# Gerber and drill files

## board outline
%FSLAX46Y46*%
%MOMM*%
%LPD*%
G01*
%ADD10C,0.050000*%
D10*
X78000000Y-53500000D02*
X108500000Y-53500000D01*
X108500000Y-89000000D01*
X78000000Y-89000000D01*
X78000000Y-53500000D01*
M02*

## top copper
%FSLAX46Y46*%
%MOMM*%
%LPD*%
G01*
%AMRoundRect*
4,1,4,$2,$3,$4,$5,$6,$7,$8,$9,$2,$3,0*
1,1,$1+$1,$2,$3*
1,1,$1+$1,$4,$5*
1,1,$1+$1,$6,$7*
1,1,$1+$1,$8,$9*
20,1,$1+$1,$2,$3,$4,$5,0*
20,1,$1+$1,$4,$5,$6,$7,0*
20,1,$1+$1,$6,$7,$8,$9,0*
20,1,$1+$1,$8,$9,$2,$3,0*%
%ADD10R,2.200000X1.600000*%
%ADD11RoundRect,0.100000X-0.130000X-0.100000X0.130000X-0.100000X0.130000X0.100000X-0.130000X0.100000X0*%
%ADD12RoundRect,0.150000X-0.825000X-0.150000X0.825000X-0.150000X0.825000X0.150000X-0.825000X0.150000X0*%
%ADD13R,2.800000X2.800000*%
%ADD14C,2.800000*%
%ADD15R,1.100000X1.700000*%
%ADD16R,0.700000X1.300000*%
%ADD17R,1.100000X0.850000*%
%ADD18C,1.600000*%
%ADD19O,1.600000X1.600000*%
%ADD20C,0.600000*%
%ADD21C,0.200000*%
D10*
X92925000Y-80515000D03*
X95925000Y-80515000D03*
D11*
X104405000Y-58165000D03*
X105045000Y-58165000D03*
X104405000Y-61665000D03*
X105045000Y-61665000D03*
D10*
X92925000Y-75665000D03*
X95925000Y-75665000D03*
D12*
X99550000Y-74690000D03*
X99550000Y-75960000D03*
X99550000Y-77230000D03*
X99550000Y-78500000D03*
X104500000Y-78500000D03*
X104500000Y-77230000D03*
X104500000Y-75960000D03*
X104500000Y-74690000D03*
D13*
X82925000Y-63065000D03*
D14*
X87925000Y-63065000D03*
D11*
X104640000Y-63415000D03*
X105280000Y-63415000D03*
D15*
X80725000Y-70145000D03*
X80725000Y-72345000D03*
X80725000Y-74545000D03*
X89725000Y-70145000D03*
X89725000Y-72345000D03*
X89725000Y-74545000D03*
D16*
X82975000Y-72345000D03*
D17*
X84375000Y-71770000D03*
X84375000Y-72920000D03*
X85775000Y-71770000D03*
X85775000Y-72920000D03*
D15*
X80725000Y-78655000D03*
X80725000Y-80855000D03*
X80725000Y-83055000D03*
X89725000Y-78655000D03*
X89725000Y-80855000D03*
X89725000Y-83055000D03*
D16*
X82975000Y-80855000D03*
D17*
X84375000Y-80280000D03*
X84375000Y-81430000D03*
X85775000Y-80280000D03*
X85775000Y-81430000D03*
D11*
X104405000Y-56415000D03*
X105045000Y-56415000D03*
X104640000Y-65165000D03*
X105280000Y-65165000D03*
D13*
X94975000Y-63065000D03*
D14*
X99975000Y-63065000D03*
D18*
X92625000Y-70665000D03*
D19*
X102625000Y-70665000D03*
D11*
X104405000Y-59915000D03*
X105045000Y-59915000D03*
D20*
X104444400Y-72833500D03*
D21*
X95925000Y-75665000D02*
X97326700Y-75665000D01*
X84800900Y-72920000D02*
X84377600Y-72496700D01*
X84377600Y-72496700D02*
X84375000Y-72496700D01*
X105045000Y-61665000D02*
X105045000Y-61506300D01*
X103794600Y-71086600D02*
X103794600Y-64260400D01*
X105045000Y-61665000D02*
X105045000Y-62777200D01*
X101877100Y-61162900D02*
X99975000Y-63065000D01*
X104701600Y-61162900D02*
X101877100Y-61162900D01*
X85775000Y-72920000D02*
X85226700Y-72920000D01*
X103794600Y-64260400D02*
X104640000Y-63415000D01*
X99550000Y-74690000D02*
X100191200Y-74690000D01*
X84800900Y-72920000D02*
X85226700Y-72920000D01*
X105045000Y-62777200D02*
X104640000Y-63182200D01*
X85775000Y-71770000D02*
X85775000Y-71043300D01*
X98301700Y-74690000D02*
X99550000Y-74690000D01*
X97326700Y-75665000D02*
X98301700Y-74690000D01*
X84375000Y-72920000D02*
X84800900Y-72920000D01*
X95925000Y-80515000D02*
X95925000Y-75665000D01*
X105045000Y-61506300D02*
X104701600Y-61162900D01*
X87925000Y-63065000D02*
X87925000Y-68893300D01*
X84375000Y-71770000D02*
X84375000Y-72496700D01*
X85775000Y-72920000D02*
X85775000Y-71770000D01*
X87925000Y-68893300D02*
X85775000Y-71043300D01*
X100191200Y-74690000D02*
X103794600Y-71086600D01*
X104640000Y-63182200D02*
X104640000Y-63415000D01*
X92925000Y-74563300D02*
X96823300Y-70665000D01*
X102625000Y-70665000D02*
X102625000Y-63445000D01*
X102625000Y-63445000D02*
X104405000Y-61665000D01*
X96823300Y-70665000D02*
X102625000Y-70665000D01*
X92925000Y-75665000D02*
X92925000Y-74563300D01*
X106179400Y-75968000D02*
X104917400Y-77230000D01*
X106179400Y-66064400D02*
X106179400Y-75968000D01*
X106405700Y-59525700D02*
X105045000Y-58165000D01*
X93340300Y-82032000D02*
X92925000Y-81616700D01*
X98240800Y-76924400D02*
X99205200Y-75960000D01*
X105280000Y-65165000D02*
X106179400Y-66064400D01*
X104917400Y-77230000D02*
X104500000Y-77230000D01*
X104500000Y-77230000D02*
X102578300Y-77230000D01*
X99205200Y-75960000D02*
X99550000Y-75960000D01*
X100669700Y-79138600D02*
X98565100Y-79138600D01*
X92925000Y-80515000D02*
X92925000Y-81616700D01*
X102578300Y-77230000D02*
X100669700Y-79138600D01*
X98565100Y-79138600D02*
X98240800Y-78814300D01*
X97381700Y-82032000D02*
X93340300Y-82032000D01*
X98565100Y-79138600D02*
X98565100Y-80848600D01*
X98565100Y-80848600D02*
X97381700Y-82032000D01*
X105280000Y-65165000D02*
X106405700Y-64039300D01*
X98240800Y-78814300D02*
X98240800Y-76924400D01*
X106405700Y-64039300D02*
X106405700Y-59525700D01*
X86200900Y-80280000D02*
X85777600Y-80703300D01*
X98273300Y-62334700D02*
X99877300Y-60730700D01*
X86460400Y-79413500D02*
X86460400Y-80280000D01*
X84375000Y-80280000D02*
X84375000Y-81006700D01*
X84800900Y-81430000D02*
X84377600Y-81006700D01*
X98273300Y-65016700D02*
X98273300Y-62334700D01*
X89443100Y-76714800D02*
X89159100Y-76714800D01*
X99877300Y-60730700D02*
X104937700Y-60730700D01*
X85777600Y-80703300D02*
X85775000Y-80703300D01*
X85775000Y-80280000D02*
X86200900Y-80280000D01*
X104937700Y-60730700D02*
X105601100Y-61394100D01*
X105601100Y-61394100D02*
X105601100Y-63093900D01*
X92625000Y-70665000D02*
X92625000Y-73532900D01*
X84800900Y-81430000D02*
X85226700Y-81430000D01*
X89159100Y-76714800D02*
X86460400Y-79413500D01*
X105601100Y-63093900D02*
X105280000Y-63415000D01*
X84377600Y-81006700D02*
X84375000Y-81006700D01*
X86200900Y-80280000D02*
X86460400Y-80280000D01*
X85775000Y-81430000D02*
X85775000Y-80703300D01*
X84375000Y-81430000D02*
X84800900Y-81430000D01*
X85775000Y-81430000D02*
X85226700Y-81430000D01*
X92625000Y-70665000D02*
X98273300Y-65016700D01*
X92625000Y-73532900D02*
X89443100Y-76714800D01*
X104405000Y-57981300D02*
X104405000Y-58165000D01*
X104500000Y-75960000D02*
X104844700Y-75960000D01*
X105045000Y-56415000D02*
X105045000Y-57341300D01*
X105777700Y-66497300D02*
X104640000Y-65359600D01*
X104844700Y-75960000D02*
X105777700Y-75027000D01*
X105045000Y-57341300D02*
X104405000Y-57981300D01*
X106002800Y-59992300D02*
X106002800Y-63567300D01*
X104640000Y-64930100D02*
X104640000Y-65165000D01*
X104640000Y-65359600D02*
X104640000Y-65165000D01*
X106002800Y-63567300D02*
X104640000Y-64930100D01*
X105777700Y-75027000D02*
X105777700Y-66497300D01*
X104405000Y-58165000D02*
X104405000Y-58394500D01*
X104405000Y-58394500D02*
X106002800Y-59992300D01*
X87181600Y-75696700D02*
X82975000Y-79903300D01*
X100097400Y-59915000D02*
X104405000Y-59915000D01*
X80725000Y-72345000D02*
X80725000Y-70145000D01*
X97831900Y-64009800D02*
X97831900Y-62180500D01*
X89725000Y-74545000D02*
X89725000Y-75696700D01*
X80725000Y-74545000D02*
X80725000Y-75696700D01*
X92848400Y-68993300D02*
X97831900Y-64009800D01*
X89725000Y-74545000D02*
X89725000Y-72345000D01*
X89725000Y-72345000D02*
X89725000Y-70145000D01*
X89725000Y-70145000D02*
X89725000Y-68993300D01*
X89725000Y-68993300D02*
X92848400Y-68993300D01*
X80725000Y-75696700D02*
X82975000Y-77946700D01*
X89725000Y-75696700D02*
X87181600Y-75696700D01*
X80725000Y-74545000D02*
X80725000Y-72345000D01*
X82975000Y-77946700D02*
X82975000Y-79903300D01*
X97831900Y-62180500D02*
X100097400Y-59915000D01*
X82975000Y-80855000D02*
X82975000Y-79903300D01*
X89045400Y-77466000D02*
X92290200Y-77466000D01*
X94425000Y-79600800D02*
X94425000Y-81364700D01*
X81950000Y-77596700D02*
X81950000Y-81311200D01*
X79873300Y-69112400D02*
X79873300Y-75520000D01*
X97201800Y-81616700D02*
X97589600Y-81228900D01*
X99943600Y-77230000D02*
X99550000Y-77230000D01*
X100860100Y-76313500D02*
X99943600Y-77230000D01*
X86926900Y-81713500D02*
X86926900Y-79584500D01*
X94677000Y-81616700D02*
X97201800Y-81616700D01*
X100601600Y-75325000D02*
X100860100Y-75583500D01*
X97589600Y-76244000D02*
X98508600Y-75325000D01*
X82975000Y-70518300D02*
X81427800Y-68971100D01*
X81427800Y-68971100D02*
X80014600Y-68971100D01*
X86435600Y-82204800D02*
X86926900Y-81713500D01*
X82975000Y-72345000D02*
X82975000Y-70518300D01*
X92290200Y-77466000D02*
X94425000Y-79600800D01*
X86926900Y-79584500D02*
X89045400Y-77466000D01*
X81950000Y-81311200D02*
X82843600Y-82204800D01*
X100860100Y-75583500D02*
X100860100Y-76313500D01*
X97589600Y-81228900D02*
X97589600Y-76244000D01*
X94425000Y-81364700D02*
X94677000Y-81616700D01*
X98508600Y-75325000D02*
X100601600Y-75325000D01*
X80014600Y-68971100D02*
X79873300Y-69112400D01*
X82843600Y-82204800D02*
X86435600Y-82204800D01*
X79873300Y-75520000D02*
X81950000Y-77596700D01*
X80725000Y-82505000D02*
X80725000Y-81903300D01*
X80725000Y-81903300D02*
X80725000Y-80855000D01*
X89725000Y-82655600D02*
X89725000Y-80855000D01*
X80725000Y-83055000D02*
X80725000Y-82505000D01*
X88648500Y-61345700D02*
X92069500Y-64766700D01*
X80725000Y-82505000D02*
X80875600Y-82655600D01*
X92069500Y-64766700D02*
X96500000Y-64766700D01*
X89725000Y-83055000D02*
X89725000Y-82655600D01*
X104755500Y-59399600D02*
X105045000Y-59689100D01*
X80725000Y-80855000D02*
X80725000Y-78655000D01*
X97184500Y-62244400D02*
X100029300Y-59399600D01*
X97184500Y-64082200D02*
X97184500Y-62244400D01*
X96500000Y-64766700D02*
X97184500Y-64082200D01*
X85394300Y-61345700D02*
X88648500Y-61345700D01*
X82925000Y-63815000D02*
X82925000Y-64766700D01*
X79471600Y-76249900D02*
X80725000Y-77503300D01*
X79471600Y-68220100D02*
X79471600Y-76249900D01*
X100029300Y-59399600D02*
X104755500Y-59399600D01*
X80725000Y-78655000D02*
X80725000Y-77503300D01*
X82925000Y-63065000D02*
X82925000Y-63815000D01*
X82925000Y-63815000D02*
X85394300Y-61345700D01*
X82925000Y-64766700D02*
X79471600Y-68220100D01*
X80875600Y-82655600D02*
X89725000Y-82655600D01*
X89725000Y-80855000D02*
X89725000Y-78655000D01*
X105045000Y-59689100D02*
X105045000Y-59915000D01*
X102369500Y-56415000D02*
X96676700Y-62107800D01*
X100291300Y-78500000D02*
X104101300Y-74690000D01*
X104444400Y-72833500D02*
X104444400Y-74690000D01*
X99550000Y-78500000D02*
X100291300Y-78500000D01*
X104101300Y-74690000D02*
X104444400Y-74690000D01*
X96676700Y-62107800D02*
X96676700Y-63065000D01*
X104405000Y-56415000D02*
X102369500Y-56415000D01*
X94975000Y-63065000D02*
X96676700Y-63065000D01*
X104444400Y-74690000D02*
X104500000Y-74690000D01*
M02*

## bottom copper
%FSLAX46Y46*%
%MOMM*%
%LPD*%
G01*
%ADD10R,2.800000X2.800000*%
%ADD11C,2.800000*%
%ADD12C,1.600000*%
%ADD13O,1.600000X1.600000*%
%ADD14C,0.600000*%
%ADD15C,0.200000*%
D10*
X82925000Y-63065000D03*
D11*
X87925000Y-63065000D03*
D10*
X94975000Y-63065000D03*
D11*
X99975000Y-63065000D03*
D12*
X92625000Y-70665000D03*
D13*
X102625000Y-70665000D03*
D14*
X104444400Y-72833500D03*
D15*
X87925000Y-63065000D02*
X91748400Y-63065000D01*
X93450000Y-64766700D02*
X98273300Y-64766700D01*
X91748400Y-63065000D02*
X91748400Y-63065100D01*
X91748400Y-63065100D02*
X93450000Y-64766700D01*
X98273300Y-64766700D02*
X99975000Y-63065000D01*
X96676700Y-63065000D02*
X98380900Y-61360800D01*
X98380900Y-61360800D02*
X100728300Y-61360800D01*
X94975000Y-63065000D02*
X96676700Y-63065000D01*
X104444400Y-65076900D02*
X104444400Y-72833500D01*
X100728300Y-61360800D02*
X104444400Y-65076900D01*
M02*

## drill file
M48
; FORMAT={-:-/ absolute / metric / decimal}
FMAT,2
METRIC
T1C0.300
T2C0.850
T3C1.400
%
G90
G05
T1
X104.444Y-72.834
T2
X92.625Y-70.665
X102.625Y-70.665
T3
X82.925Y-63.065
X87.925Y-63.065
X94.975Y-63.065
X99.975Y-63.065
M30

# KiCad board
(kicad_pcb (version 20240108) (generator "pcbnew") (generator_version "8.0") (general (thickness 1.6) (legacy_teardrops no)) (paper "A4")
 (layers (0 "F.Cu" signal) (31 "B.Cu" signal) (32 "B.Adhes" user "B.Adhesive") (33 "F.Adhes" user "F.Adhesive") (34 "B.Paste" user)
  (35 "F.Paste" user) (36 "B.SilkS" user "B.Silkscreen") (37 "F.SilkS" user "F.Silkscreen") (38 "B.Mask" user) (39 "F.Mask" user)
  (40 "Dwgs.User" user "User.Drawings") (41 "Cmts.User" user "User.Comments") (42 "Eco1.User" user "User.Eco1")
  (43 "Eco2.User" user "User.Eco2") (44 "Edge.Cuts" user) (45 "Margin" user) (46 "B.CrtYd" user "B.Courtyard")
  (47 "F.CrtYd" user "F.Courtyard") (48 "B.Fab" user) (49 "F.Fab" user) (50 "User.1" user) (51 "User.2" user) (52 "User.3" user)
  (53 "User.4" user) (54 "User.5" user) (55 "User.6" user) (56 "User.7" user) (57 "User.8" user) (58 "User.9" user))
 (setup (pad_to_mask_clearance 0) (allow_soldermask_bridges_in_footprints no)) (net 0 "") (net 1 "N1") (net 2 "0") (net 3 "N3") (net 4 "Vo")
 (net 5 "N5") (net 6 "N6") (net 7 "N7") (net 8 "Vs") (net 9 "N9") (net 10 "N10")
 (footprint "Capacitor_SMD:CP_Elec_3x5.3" (layer "F.Cu") (at 94.425 80.515)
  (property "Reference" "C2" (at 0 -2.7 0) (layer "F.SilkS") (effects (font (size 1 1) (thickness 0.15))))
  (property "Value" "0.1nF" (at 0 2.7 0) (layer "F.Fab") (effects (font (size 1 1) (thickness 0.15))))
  (pad "1" smd rect (at -1.5 0) (size 2.2 1.6) (layers "F.Cu" "F.Paste" "F.Mask") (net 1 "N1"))
  (pad "2" smd rect (at 1.5 0) (size 2.2 1.6) (layers "F.Cu" "F.Paste" "F.Mask") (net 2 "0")))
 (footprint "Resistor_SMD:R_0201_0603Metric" (layer "F.Cu") (at 104.725 58.165)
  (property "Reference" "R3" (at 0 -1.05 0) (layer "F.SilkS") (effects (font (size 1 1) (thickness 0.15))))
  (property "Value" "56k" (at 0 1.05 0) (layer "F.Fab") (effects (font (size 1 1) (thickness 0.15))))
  (pad "" smd roundrect (at -0.345 0) (size 0.318 0.36) (layers "F.Paste") (roundrect_rratio 0.25))
  (pad "" smd roundrect (at 0.345 0) (size 0.318 0.36) (layers "F.Paste") (roundrect_rratio 0.25))
  (pad "1" smd roundrect (at -0.32 0) (size 0.46 0.4) (layers "F.Cu" "F.Mask") (roundrect_rratio 0.25) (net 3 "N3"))
  (pad "2" smd roundrect (at 0.32 0) (size 0.46 0.4) (layers "F.Cu" "F.Mask") (roundrect_rratio 0.25) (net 1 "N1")))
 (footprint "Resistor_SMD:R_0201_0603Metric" (layer "F.Cu") (at 104.725 61.665)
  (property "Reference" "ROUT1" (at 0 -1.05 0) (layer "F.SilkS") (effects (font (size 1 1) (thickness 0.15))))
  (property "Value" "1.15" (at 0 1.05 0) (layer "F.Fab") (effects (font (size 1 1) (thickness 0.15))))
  (pad "" smd roundrect (at -0.345 0) (size 0.318 0.36) (layers "F.Paste") (roundrect_rratio 0.25))
  (pad "" smd roundrect (at 0.345 0) (size 0.318 0.36) (layers "F.Paste") (roundrect_rratio 0.25))
  (pad "1" smd roundrect (at -0.32 0) (size 0.46 0.4) (layers "F.Cu" "F.Mask") (roundrect_rratio 0.25) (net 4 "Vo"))
  (pad "2" smd roundrect (at 0.32 0) (size 0.46 0.4) (layers "F.Cu" "F.Mask") (roundrect_rratio 0.25) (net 2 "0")))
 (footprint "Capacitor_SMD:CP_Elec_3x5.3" (layer "F.Cu") (at 94.425 75.665)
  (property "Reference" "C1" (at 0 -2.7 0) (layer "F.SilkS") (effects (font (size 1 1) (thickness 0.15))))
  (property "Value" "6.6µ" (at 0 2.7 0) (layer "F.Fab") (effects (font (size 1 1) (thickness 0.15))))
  (pad "1" smd rect (at -1.5 0) (size 2.2 1.6) (layers "F.Cu" "F.Paste" "F.Mask") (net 4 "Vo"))
  (pad "2" smd rect (at 1.5 0) (size 2.2 1.6) (layers "F.Cu" "F.Paste" "F.Mask") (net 2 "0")))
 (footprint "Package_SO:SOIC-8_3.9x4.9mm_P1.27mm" (layer "F.Cu") (at 102.025 76.595)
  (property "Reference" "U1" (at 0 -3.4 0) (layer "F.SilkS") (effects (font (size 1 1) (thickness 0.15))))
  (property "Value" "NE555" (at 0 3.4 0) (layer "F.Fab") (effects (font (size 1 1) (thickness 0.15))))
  (pad "1" smd roundrect (at -2.475 -1.905) (size 1.95 0.6) (layers "F.Cu" "F.Paste" "F.Mask") (roundrect_rratio 0.25) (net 2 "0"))
  (pad "2" smd roundrect (at -2.475 -0.635) (size 1.95 0.6) (layers "F.Cu" "F.Paste" "F.Mask") (roundrect_rratio 0.25) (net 1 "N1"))
  (pad "3" smd roundrect (at -2.475 0.635) (size 1.95 0.6) (layers "F.Cu" "F.Paste" "F.Mask") (roundrect_rratio 0.25) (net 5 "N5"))
  (pad "4" smd roundrect (at -2.475 1.905) (size 1.95 0.6) (layers "F.Cu" "F.Paste" "F.Mask") (roundrect_rratio 0.25) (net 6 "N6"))
  (pad "5" smd roundrect (at 2.475 1.905) (size 1.95 0.6) (layers "F.Cu" "F.Paste" "F.Mask") (roundrect_rratio 0.25) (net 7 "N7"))
  (pad "6" smd roundrect (at 2.475 0.635) (size 1.95 0.6) (layers "F.Cu" "F.Paste" "F.Mask") (roundrect_rratio 0.25) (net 1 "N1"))
  (pad "7" smd roundrect (at 2.475 -0.635) (size 1.95 0.6) (layers "F.Cu" "F.Paste" "F.Mask") (roundrect_rratio 0.25) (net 3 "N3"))
  (pad "8" smd roundrect (at 2.475 -1.905) (size 1.95 0.6) (layers "F.Cu" "F.Paste" "F.Mask") (roundrect_rratio 0.25) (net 6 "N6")))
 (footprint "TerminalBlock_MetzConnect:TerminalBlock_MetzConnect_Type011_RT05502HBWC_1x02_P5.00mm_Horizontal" (layer "F.Cu")
  (at 82.925 63.065)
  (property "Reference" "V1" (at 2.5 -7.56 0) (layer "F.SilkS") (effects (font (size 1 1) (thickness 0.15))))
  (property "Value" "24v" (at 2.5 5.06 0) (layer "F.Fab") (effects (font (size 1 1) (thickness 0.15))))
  (pad "1" thru_hole rect (at 0 0) (size 2.8 2.8) (drill 1.4) (layers "*.Cu" "*.Mask") (remove_unused_layers no) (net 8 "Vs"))
  (pad "2" thru_hole circle (at 5 0) (size 2.8 2.8) (drill 1.4) (layers "*.Cu" "*.Mask") (remove_unused_layers no) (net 2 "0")))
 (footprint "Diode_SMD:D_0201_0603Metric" (layer "F.Cu") (at 104.96 63.415)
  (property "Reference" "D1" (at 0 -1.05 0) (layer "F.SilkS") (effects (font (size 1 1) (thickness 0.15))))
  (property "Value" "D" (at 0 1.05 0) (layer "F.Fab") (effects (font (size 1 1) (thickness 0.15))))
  (pad "" smd roundrect (at -0.345 0) (size 0.318 0.36) (layers "F.Paste") (roundrect_rratio 0.25))
  (pad "" smd roundrect (at 0.345 0) (size 0.318 0.36) (layers "F.Paste") (roundrect_rratio 0.25))
  (pad "1" smd roundrect (at -0.32 0) (size 0.46 0.4) (layers "F.Cu" "F.Mask") (roundrect_rratio 0.25) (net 2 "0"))
  (pad "2" smd roundrect (at 0.32 0) (size 0.46 0.4) (layers "F.Cu" "F.Mask") (roundrect_rratio 0.25) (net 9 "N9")))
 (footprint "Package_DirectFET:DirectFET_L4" (layer "F.Cu") (at 85.225 72.345)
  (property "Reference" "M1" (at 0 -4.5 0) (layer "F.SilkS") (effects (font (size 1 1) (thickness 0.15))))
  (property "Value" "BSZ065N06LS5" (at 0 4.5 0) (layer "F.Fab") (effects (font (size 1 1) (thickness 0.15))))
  (pad "1" smd rect (at -4.5 -2.2) (size 1.1 1.7) (layers "F.Cu" "F.Paste" "F.Mask") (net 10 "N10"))
  (pad "1" smd rect (at -4.5 0) (size 1.1 1.7) (layers "F.Cu" "F.Paste" "F.Mask") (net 10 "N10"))
  (pad "1" smd rect (at -4.5 2.2) (size 1.1 1.7) (layers "F.Cu" "F.Paste" "F.Mask") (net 10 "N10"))
  (pad "1" smd rect (at 4.5 -2.2) (size 1.1 1.7) (layers "F.Cu" "F.Paste" "F.Mask") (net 10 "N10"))
  (pad "1" smd rect (at 4.5 0) (size 1.1 1.7) (layers "F.Cu" "F.Paste" "F.Mask") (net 10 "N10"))
  (pad "1" smd rect (at 4.5 2.2) (size 1.1 1.7) (layers "F.Cu" "F.Paste" "F.Mask") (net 10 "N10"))
  (pad "2" smd rect (at -2.25 0) (size 0.7 1.3) (layers "F.Cu" "F.Paste" "F.Mask") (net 5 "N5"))
  (pad "3" smd rect (at -0.85 -0.575) (size 1.1 0.85) (layers "F.Cu" "F.Paste" "F.Mask") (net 2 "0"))
  (pad "3" smd rect (at -0.85 0.575) (size 1.1 0.85) (layers "F.Cu" "F.Paste" "F.Mask") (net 2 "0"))
  (pad "3" smd rect (at 0.55 -0.575) (size 1.1 0.85) (layers "F.Cu" "F.Paste" "F.Mask") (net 2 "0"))
  (pad "3" smd rect (at 0.55 0.575) (size 1.1 0.85) (layers "F.Cu" "F.Paste" "F.Mask") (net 2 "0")))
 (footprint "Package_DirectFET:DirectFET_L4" (layer "F.Cu") (at 85.225 80.855)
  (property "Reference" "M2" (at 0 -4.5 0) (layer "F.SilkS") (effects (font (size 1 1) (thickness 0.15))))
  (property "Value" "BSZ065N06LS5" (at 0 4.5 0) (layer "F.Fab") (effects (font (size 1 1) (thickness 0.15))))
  (pad "1" smd rect (at -4.5 -2.2) (size 1.1 1.7) (layers "F.Cu" "F.Paste" "F.Mask") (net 8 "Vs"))
  (pad "1" smd rect (at -4.5 0) (size 1.1 1.7) (layers "F.Cu" "F.Paste" "F.Mask") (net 8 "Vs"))
  (pad "1" smd rect (at -4.5 2.2) (size 1.1 1.7) (layers "F.Cu" "F.Paste" "F.Mask") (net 8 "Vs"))
  (pad "1" smd rect (at 4.5 -2.2) (size 1.1 1.7) (layers "F.Cu" "F.Paste" "F.Mask") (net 8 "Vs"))
  (pad "1" smd rect (at 4.5 0) (size 1.1 1.7) (layers "F.Cu" "F.Paste" "F.Mask") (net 8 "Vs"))
  (pad "1" smd rect (at 4.5 2.2) (size 1.1 1.7) (layers "F.Cu" "F.Paste" "F.Mask") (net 8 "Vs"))
  (pad "2" smd rect (at -2.25 0) (size 0.7 1.3) (layers "F.Cu" "F.Paste" "F.Mask") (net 10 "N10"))
  (pad "3" smd rect (at -0.85 -0.575) (size 1.1 0.85) (layers "F.Cu" "F.Paste" "F.Mask") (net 9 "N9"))
  (pad "3" smd rect (at -0.85 0.575) (size 1.1 0.85) (layers "F.Cu" "F.Paste" "F.Mask") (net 9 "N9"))
  (pad "3" smd rect (at 0.55 -0.575) (size 1.1 0.85) (layers "F.Cu" "F.Paste" "F.Mask") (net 9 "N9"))
  (pad "3" smd rect (at 0.55 0.575) (size 1.1 0.85) (layers "F.Cu" "F.Paste" "F.Mask") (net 9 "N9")))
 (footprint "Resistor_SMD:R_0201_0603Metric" (layer "F.Cu") (at 104.725 56.415)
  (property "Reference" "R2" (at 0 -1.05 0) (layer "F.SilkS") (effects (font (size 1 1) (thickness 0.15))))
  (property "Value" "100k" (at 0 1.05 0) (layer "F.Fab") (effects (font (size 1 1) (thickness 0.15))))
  (pad "" smd roundrect (at -0.345 0) (size 0.318 0.36) (layers "F.Paste") (roundrect_rratio 0.25))
  (pad "" smd roundrect (at 0.345 0) (size 0.318 0.36) (layers "F.Paste") (roundrect_rratio 0.25))
  (pad "1" smd roundrect (at -0.32 0) (size 0.46 0.4) (layers "F.Cu" "F.Mask") (roundrect_rratio 0.25) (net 6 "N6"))
  (pad "2" smd roundrect (at 0.32 0) (size 0.46 0.4) (layers "F.Cu" "F.Mask") (roundrect_rratio 0.25) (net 3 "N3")))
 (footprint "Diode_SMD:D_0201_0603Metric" (layer "F.Cu") (at 104.96 65.165)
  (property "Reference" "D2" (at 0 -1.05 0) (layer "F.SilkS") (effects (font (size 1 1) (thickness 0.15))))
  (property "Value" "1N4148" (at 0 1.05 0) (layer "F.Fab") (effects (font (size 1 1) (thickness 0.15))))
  (pad "" smd roundrect (at -0.345 0) (size 0.318 0.36) (layers "F.Paste") (roundrect_rratio 0.25))
  (pad "" smd roundrect (at 0.345 0) (size 0.318 0.36) (layers "F.Paste") (roundrect_rratio 0.25))
  (pad "1" smd roundrect (at -0.32 0) (size 0.46 0.4) (layers "F.Cu" "F.Mask") (roundrect_rratio 0.25) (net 3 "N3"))
  (pad "2" smd roundrect (at 0.32 0) (size 0.46 0.4) (layers "F.Cu" "F.Mask") (roundrect_rratio 0.25) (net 1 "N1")))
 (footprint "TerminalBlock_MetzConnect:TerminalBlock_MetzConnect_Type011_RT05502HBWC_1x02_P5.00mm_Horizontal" (layer "F.Cu")
  (at 94.975 63.065)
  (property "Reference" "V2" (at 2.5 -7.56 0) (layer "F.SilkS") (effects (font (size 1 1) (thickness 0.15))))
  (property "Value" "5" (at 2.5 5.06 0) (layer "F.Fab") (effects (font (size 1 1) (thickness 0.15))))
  (pad "1" thru_hole rect (at 0 0) (size 2.8 2.8) (drill 1.4) (layers "*.Cu" "*.Mask") (remove_unused_layers no) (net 6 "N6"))
  (pad "2" thru_hole circle (at 5 0) (size 2.8 2.8) (drill 1.4) (layers "*.Cu" "*.Mask") (remove_unused_layers no) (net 2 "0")))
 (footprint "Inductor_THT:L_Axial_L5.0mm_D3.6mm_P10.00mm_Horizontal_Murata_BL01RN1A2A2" (layer "F.Cu") (at 92.625 70.665)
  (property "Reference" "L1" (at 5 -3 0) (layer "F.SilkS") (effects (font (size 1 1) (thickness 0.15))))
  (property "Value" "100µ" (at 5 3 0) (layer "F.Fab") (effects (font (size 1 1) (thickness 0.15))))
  (pad "1" thru_hole circle (at 0 0) (size 1.6 1.6) (drill 0.85) (layers "*.Cu" "*.Mask") (remove_unused_layers no) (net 9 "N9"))
  (pad "2" thru_hole oval (at 10 0) (size 1.6 1.6) (drill 0.85) (layers "*.Cu" "*.Mask") (remove_unused_layers no) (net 4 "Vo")))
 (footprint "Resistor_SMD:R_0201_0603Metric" (layer "F.Cu") (at 104.725 59.915)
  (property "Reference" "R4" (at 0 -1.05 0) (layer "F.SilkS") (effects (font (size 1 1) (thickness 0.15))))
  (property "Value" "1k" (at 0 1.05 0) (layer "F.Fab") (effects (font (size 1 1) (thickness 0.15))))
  (pad "" smd roundrect (at -0.345 0) (size 0.318 0.36) (layers "F.Paste") (roundrect_rratio 0.25))
  (pad "" smd roundrect (at 0.345 0) (size 0.318 0.36) (layers "F.Paste") (roundrect_rratio 0.25))
  (pad "1" smd roundrect (at -0.32 0) (size 0.46 0.4) (layers "F.Cu" "F.Mask") (roundrect_rratio 0.25) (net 10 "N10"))
  (pad "2" smd roundrect (at 0.32 0) (size 0.46 0.4) (layers "F.Cu" "F.Mask") (roundrect_rratio 0.25) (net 8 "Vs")))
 (gr_rect (start 78 53.5) (end 108.5 89) (stroke (width 0.05) (type default)) (fill none) (layer "Edge.Cuts"))
 (segment (start 95.925 75.665) (end 97.3267 75.665) (width 0.2) (layer "F.Cu") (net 2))
 (segment (start 84.8009 72.92) (end 84.3776 72.4967) (width 0.2) (layer "F.Cu") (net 2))
 (segment (start 84.3776 72.4967) (end 84.375 72.4967) (width 0.2) (layer "F.Cu") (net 2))
 (segment (start 105.045 61.665) (end 105.045 61.5063) (width 0.2) (layer "F.Cu") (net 2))
 (segment (start 103.7946 71.0866) (end 103.7946 64.2604) (width 0.2) (layer "F.Cu") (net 2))
 (segment (start 105.045 61.665) (end 105.045 62.7772) (width 0.2) (layer "F.Cu") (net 2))
 (segment (start 101.8771 61.1629) (end 99.975 63.065) (width 0.2) (layer "F.Cu") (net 2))
 (segment (start 104.7016 61.1629) (end 101.8771 61.1629) (width 0.2) (layer "F.Cu") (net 2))
 (segment (start 85.775 72.92) (end 85.2267 72.92) (width 0.2) (layer "F.Cu") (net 2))
 (segment (start 103.7946 64.2604) (end 104.64 63.415) (width 0.2) (layer "F.Cu") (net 2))
 (segment (start 99.55 74.69) (end 100.1912 74.69) (width 0.2) (layer "F.Cu") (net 2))
 (segment (start 84.8009 72.92) (end 85.2267 72.92) (width 0.2) (layer "F.Cu") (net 2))
 (segment (start 105.045 62.7772) (end 104.64 63.1822) (width 0.2) (layer "F.Cu") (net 2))
 (segment (start 85.775 71.77) (end 85.775 71.0433) (width 0.2) (layer "F.Cu") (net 2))
 (segment (start 98.3017 74.69) (end 99.55 74.69) (width 0.2) (layer "F.Cu") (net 2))
 (segment (start 97.3267 75.665) (end 98.3017 74.69) (width 0.2) (layer "F.Cu") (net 2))
 (segment (start 84.375 72.92) (end 84.8009 72.92) (width 0.2) (layer "F.Cu") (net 2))
 (segment (start 95.925 80.515) (end 95.925 75.665) (width 0.2) (layer "F.Cu") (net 2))
 (segment (start 105.045 61.5063) (end 104.7016 61.1629) (width 0.2) (layer "F.Cu") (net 2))
 (segment (start 87.925 63.065) (end 87.925 68.8933) (width 0.2) (layer "F.Cu") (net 2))
 (segment (start 84.375 71.77) (end 84.375 72.4967) (width 0.2) (layer "F.Cu") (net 2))
 (segment (start 85.775 72.92) (end 85.775 71.77) (width 0.2) (layer "F.Cu") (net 2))
 (segment (start 87.925 68.8933) (end 85.775 71.0433) (width 0.2) (layer "F.Cu") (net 2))
 (segment (start 100.1912 74.69) (end 103.7946 71.0866) (width 0.2) (layer "F.Cu") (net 2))
 (segment (start 104.64 63.1822) (end 104.64 63.415) (width 0.2) (layer "F.Cu") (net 2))
 (segment (start 87.925 63.065) (end 91.7484 63.065) (width 0.2) (layer "B.Cu") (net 2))
 (segment (start 93.45 64.7667) (end 98.2733 64.7667) (width 0.2) (layer "B.Cu") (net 2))
 (segment (start 91.7484 63.065) (end 91.7484 63.0651) (width 0.2) (layer "B.Cu") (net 2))
 (segment (start 91.7484 63.0651) (end 93.45 64.7667) (width 0.2) (layer "B.Cu") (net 2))
 (segment (start 98.2733 64.7667) (end 99.975 63.065) (width 0.2) (layer "B.Cu") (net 2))
 (segment (start 92.925 74.5633) (end 96.8233 70.665) (width 0.2) (layer "F.Cu") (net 4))
 (segment (start 102.625 70.665) (end 102.625 63.445) (width 0.2) (layer "F.Cu") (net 4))
 (segment (start 102.625 63.445) (end 104.405 61.665) (width 0.2) (layer "F.Cu") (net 4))
 (segment (start 96.8233 70.665) (end 102.625 70.665) (width 0.2) (layer "F.Cu") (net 4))
 (segment (start 92.925 75.665) (end 92.925 74.5633) (width 0.2) (layer "F.Cu") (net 4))
 (segment (start 106.1794 75.968) (end 104.9174 77.23) (width 0.2) (layer "F.Cu") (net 1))
 (segment (start 106.1794 66.0644) (end 106.1794 75.968) (width 0.2) (layer "F.Cu") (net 1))
 (segment (start 106.4057 59.5257) (end 105.045 58.165) (width 0.2) (layer "F.Cu") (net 1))
 (segment (start 93.3403 82.032) (end 92.925 81.6167) (width 0.2) (layer "F.Cu") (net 1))
 (segment (start 98.2408 76.9244) (end 99.2052 75.96) (width 0.2) (layer "F.Cu") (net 1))
 (segment (start 105.28 65.165) (end 106.1794 66.0644) (width 0.2) (layer "F.Cu") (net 1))
 (segment (start 104.9174 77.23) (end 104.5 77.23) (width 0.2) (layer "F.Cu") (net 1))
 (segment (start 104.5 77.23) (end 102.5783 77.23) (width 0.2) (layer "F.Cu") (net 1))
 (segment (start 99.2052 75.96) (end 99.55 75.96) (width 0.2) (layer "F.Cu") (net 1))
 (segment (start 100.6697 79.1386) (end 98.5651 79.1386) (width 0.2) (layer "F.Cu") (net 1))
 (segment (start 92.925 80.515) (end 92.925 81.6167) (width 0.2) (layer "F.Cu") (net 1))
 (segment (start 102.5783 77.23) (end 100.6697 79.1386) (width 0.2) (layer "F.Cu") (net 1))
 (segment (start 98.5651 79.1386) (end 98.2408 78.8143) (width 0.2) (layer "F.Cu") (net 1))
 (segment (start 97.3817 82.032) (end 93.3403 82.032) (width 0.2) (layer "F.Cu") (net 1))
 (segment (start 98.5651 79.1386) (end 98.5651 80.8486) (width 0.2) (layer "F.Cu") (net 1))
 (segment (start 98.5651 80.8486) (end 97.3817 82.032) (width 0.2) (layer "F.Cu") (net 1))
 (segment (start 105.28 65.165) (end 106.4057 64.0393) (width 0.2) (layer "F.Cu") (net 1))
 (segment (start 98.2408 78.8143) (end 98.2408 76.9244) (width 0.2) (layer "F.Cu") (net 1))
 (segment (start 106.4057 64.0393) (end 106.4057 59.5257) (width 0.2) (layer "F.Cu") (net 1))
 (segment (start 86.2009 80.28) (end 85.7776 80.7033) (width 0.2) (layer "F.Cu") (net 9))
 (segment (start 98.2733 62.3347) (end 99.8773 60.7307) (width 0.2) (layer "F.Cu") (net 9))
 (segment (start 86.4604 79.4135) (end 86.4604 80.28) (width 0.2) (layer "F.Cu") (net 9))
 (segment (start 84.375 80.28) (end 84.375 81.0067) (width 0.2) (layer "F.Cu") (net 9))
 (segment (start 84.8009 81.43) (end 84.3776 81.0067) (width 0.2) (layer "F.Cu") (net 9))
 (segment (start 98.2733 65.0167) (end 98.2733 62.3347) (width 0.2) (layer "F.Cu") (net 9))
 (segment (start 89.4431 76.7148) (end 89.1591 76.7148) (width 0.2) (layer "F.Cu") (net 9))
 (segment (start 99.8773 60.7307) (end 104.9377 60.7307) (width 0.2) (layer "F.Cu") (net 9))
 (segment (start 85.7776 80.7033) (end 85.775 80.7033) (width 0.2) (layer "F.Cu") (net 9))
 (segment (start 85.775 80.28) (end 86.2009 80.28) (width 0.2) (layer "F.Cu") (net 9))
 (segment (start 104.9377 60.7307) (end 105.6011 61.3941) (width 0.2) (layer "F.Cu") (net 9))
 (segment (start 105.6011 61.3941) (end 105.6011 63.0939) (width 0.2) (layer "F.Cu") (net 9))
 (segment (start 92.625 70.665) (end 92.625 73.5329) (width 0.2) (layer "F.Cu") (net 9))
 (segment (start 84.8009 81.43) (end 85.2267 81.43) (width 0.2) (layer "F.Cu") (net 9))
 (segment (start 89.1591 76.7148) (end 86.4604 79.4135) (width 0.2) (layer "F.Cu") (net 9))
 (segment (start 105.6011 63.0939) (end 105.28 63.415) (width 0.2) (layer "F.Cu") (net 9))
 (segment (start 84.3776 81.0067) (end 84.375 81.0067) (width 0.2) (layer "F.Cu") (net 9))
 (segment (start 86.2009 80.28) (end 86.4604 80.28) (width 0.2) (layer "F.Cu") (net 9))
 (segment (start 85.775 81.43) (end 85.775 80.7033) (width 0.2) (layer "F.Cu") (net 9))
 (segment (start 84.375 81.43) (end 84.8009 81.43) (width 0.2) (layer "F.Cu") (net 9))
 (segment (start 85.775 81.43) (end 85.2267 81.43) (width 0.2) (layer "F.Cu") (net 9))
 (segment (start 92.625 70.665) (end 98.2733 65.0167) (width 0.2) (layer "F.Cu") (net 9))
 (segment (start 92.625 73.5329) (end 89.4431 76.7148) (width 0.2) (layer "F.Cu") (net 9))
 (segment (start 104.405 57.9813) (end 104.405 58.165) (width 0.2) (layer "F.Cu") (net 3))
 (segment (start 104.5 75.96) (end 104.8447 75.96) (width 0.2) (layer "F.Cu") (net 3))
 (segment (start 105.045 56.415) (end 105.045 57.3413) (width 0.2) (layer "F.Cu") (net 3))
 (segment (start 105.7777 66.4973) (end 104.64 65.3596) (width 0.2) (layer "F.Cu") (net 3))
 (segment (start 104.8447 75.96) (end 105.7777 75.027) (width 0.2) (layer "F.Cu") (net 3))
 (segment (start 105.045 57.3413) (end 104.405 57.9813) (width 0.2) (layer "F.Cu") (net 3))
 (segment (start 106.0028 59.9923) (end 106.0028 63.5673) (width 0.2) (layer "F.Cu") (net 3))
 (segment (start 104.64 64.9301) (end 104.64 65.165) (width 0.2) (layer "F.Cu") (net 3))
 (segment (start 104.64 65.3596) (end 104.64 65.165) (width 0.2) (layer "F.Cu") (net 3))
 (segment (start 106.0028 63.5673) (end 104.64 64.9301) (width 0.2) (layer "F.Cu") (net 3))
 (segment (start 105.7777 75.027) (end 105.7777 66.4973) (width 0.2) (layer "F.Cu") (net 3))
 (segment (start 104.405 58.165) (end 104.405 58.3945) (width 0.2) (layer "F.Cu") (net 3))
 (segment (start 104.405 58.3945) (end 106.0028 59.9923) (width 0.2) (layer "F.Cu") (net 3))
 (segment (start 87.1816 75.6967) (end 82.975 79.9033) (width 0.2) (layer "F.Cu") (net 10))
 (segment (start 100.0974 59.915) (end 104.405 59.915) (width 0.2) (layer "F.Cu") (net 10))
 (segment (start 80.725 72.345) (end 80.725 70.145) (width 0.2) (layer "F.Cu") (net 10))
 (segment (start 97.8319 64.0098) (end 97.8319 62.1805) (width 0.2) (layer "F.Cu") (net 10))
 (segment (start 89.725 74.545) (end 89.725 75.6967) (width 0.2) (layer "F.Cu") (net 10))
 (segment (start 80.725 74.545) (end 80.725 75.6967) (width 0.2) (layer "F.Cu") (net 10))
 (segment (start 92.8484 68.9933) (end 97.8319 64.0098) (width 0.2) (layer "F.Cu") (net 10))
 (segment (start 89.725 74.545) (end 89.725 72.345) (width 0.2) (layer "F.Cu") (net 10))
 (segment (start 89.725 72.345) (end 89.725 70.145) (width 0.2) (layer "F.Cu") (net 10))
 (segment (start 89.725 70.145) (end 89.725 68.9933) (width 0.2) (layer "F.Cu") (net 10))
 (segment (start 89.725 68.9933) (end 92.8484 68.9933) (width 0.2) (layer "F.Cu") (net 10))
 (segment (start 80.725 75.6967) (end 82.975 77.9467) (width 0.2) (layer "F.Cu") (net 10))
 (segment (start 89.725 75.6967) (end 87.1816 75.6967) (width 0.2) (layer "F.Cu") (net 10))
 (segment (start 80.725 74.545) (end 80.725 72.345) (width 0.2) (layer "F.Cu") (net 10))
 (segment (start 82.975 77.9467) (end 82.975 79.9033) (width 0.2) (layer "F.Cu") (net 10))
 (segment (start 97.8319 62.1805) (end 100.0974 59.915) (width 0.2) (layer "F.Cu") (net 10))
 (segment (start 82.975 80.855) (end 82.975 79.9033) (width 0.2) (layer "F.Cu") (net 10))
 (segment (start 89.0454 77.466) (end 92.2902 77.466) (width 0.2) (layer "F.Cu") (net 5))
 (segment (start 94.425 79.6008) (end 94.425 81.3647) (width 0.2) (layer "F.Cu") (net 5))
 (segment (start 81.95 77.5967) (end 81.95 81.3112) (width 0.2) (layer "F.Cu") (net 5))
 (segment (start 79.8733 69.1124) (end 79.8733 75.52) (width 0.2) (layer "F.Cu") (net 5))
 (segment (start 97.2018 81.6167) (end 97.5896 81.2289) (width 0.2) (layer "F.Cu") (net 5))
 (segment (start 99.9436 77.23) (end 99.55 77.23) (width 0.2) (layer "F.Cu") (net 5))
 (segment (start 100.8601 76.3135) (end 99.9436 77.23) (width 0.2) (layer "F.Cu") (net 5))
 (segment (start 86.9269 81.7135) (end 86.9269 79.5845) (width 0.2) (layer "F.Cu") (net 5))
 (segment (start 94.677 81.6167) (end 97.2018 81.6167) (width 0.2) (layer "F.Cu") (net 5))
 (segment (start 100.6016 75.325) (end 100.8601 75.5835) (width 0.2) (layer "F.Cu") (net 5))
 (segment (start 97.5896 76.244) (end 98.5086 75.325) (width 0.2) (layer "F.Cu") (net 5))
 (segment (start 82.975 70.5183) (end 81.4278 68.9711) (width 0.2) (layer "F.Cu") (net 5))
 (segment (start 81.4278 68.9711) (end 80.0146 68.9711) (width 0.2) (layer "F.Cu") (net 5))
 (segment (start 86.4356 82.2048) (end 86.9269 81.7135) (width 0.2) (layer "F.Cu") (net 5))
 (segment (start 82.975 72.345) (end 82.975 70.5183) (width 0.2) (layer "F.Cu") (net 5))
 (segment (start 92.2902 77.466) (end 94.425 79.6008) (width 0.2) (layer "F.Cu") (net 5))
 (segment (start 86.9269 79.5845) (end 89.0454 77.466) (width 0.2) (layer "F.Cu") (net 5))
 (segment (start 81.95 81.3112) (end 82.8436 82.2048) (width 0.2) (layer "F.Cu") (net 5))
 (segment (start 100.8601 75.5835) (end 100.8601 76.3135) (width 0.2) (layer "F.Cu") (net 5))
 (segment (start 97.5896 81.2289) (end 97.5896 76.244) (width 0.2) (layer "F.Cu") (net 5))
 (segment (start 94.425 81.3647) (end 94.677 81.6167) (width 0.2) (layer "F.Cu") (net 5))
 (segment (start 98.5086 75.325) (end 100.6016 75.325) (width 0.2) (layer "F.Cu") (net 5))
 (segment (start 80.0146 68.9711) (end 79.8733 69.1124) (width 0.2) (layer "F.Cu") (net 5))
 (segment (start 82.8436 82.2048) (end 86.4356 82.2048) (width 0.2) (layer "F.Cu") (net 5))
 (segment (start 79.8733 75.52) (end 81.95 77.5967) (width 0.2) (layer "F.Cu") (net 5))
 (segment (start 80.725 82.505) (end 80.725 81.9033) (width 0.2) (layer "F.Cu") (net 8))
 (segment (start 80.725 81.9033) (end 80.725 80.855) (width 0.2) (layer "F.Cu") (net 8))
 (segment (start 89.725 82.6556) (end 89.725 80.855) (width 0.2) (layer "F.Cu") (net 8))
 (segment (start 80.725 83.055) (end 80.725 82.505) (width 0.2) (layer "F.Cu") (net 8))
 (segment (start 88.6485 61.3457) (end 92.0695 64.7667) (width 0.2) (layer "F.Cu") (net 8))
 (segment (start 80.725 82.505) (end 80.8756 82.6556) (width 0.2) (layer "F.Cu") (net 8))
 (segment (start 92.0695 64.7667) (end 96.5 64.7667) (width 0.2) (layer "F.Cu") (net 8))
 (segment (start 89.725 83.055) (end 89.725 82.6556) (width 0.2) (layer "F.Cu") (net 8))
 (segment (start 104.7555 59.3996) (end 105.045 59.6891) (width 0.2) (layer "F.Cu") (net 8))
 (segment (start 80.725 80.855) (end 80.725 78.655) (width 0.2) (layer "F.Cu") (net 8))
 (segment (start 97.1845 62.2444) (end 100.0293 59.3996) (width 0.2) (layer "F.Cu") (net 8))
 (segment (start 97.1845 64.0822) (end 97.1845 62.2444) (width 0.2) (layer "F.Cu") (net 8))
 (segment (start 96.5 64.7667) (end 97.1845 64.0822) (width 0.2) (layer "F.Cu") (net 8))
 (segment (start 85.3943 61.3457) (end 88.6485 61.3457) (width 0.2) (layer "F.Cu") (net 8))
 (segment (start 82.925 63.815) (end 82.925 64.7667) (width 0.2) (layer "F.Cu") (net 8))
 (segment (start 79.4716 76.2499) (end 80.725 77.5033) (width 0.2) (layer "F.Cu") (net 8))
 (segment (start 79.4716 68.2201) (end 79.4716 76.2499) (width 0.2) (layer "F.Cu") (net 8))
 (segment (start 100.0293 59.3996) (end 104.7555 59.3996) (width 0.2) (layer "F.Cu") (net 8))
 (segment (start 80.725 78.655) (end 80.725 77.5033) (width 0.2) (layer "F.Cu") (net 8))
 (segment (start 82.925 63.065) (end 82.925 63.815) (width 0.2) (layer "F.Cu") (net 8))
 (segment (start 82.925 63.815) (end 85.3943 61.3457) (width 0.2) (layer "F.Cu") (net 8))
 (segment (start 82.925 64.7667) (end 79.4716 68.2201) (width 0.2) (layer "F.Cu") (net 8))
 (segment (start 80.8756 82.6556) (end 89.725 82.6556) (width 0.2) (layer "F.Cu") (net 8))
 (segment (start 89.725 80.855) (end 89.725 78.655) (width 0.2) (layer "F.Cu") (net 8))
 (segment (start 105.045 59.6891) (end 105.045 59.915) (width 0.2) (layer "F.Cu") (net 8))
 (segment (start 102.3695 56.415) (end 96.6767 62.1078) (width 0.2) (layer "F.Cu") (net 6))
 (segment (start 100.2913 78.5) (end 104.1013 74.69) (width 0.2) (layer "F.Cu") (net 6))
 (segment (start 104.4444 72.8335) (end 104.4444 74.69) (width 0.2) (layer "F.Cu") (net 6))
 (segment (start 99.55 78.5) (end 100.2913 78.5) (width 0.2) (layer "F.Cu") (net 6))
 (segment (start 104.1013 74.69) (end 104.4444 74.69) (width 0.2) (layer "F.Cu") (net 6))
 (segment (start 96.6767 62.1078) (end 96.6767 63.065) (width 0.2) (layer "F.Cu") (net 6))
 (segment (start 104.405 56.415) (end 102.3695 56.415) (width 0.2) (layer "F.Cu") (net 6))
 (segment (start 94.975 63.065) (end 96.6767 63.065) (width 0.2) (layer "F.Cu") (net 6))
 (segment (start 104.4444 74.69) (end 104.5 74.69) (width 0.2) (layer "F.Cu") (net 6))
 (via (at 104.4444 72.8335) (size 0.6) (drill 0.3) (layers "F.Cu" "B.Cu") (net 6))
 (segment (start 96.6767 63.065) (end 98.3809 61.3608) (width 0.2) (layer "B.Cu") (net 6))
 (segment (start 98.3809 61.3608) (end 100.7283 61.3608) (width 0.2) (layer "B.Cu") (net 6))
 (segment (start 94.975 63.065) (end 96.6767 63.065) (width 0.2) (layer "B.Cu") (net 6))
 (segment (start 104.4444 65.0769) (end 104.4444 72.8335) (width 0.2) (layer "B.Cu") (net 6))
 (segment (start 100.7283 61.3608) (end 104.4444 65.0769) (width 0.2) (layer "B.Cu") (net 6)))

